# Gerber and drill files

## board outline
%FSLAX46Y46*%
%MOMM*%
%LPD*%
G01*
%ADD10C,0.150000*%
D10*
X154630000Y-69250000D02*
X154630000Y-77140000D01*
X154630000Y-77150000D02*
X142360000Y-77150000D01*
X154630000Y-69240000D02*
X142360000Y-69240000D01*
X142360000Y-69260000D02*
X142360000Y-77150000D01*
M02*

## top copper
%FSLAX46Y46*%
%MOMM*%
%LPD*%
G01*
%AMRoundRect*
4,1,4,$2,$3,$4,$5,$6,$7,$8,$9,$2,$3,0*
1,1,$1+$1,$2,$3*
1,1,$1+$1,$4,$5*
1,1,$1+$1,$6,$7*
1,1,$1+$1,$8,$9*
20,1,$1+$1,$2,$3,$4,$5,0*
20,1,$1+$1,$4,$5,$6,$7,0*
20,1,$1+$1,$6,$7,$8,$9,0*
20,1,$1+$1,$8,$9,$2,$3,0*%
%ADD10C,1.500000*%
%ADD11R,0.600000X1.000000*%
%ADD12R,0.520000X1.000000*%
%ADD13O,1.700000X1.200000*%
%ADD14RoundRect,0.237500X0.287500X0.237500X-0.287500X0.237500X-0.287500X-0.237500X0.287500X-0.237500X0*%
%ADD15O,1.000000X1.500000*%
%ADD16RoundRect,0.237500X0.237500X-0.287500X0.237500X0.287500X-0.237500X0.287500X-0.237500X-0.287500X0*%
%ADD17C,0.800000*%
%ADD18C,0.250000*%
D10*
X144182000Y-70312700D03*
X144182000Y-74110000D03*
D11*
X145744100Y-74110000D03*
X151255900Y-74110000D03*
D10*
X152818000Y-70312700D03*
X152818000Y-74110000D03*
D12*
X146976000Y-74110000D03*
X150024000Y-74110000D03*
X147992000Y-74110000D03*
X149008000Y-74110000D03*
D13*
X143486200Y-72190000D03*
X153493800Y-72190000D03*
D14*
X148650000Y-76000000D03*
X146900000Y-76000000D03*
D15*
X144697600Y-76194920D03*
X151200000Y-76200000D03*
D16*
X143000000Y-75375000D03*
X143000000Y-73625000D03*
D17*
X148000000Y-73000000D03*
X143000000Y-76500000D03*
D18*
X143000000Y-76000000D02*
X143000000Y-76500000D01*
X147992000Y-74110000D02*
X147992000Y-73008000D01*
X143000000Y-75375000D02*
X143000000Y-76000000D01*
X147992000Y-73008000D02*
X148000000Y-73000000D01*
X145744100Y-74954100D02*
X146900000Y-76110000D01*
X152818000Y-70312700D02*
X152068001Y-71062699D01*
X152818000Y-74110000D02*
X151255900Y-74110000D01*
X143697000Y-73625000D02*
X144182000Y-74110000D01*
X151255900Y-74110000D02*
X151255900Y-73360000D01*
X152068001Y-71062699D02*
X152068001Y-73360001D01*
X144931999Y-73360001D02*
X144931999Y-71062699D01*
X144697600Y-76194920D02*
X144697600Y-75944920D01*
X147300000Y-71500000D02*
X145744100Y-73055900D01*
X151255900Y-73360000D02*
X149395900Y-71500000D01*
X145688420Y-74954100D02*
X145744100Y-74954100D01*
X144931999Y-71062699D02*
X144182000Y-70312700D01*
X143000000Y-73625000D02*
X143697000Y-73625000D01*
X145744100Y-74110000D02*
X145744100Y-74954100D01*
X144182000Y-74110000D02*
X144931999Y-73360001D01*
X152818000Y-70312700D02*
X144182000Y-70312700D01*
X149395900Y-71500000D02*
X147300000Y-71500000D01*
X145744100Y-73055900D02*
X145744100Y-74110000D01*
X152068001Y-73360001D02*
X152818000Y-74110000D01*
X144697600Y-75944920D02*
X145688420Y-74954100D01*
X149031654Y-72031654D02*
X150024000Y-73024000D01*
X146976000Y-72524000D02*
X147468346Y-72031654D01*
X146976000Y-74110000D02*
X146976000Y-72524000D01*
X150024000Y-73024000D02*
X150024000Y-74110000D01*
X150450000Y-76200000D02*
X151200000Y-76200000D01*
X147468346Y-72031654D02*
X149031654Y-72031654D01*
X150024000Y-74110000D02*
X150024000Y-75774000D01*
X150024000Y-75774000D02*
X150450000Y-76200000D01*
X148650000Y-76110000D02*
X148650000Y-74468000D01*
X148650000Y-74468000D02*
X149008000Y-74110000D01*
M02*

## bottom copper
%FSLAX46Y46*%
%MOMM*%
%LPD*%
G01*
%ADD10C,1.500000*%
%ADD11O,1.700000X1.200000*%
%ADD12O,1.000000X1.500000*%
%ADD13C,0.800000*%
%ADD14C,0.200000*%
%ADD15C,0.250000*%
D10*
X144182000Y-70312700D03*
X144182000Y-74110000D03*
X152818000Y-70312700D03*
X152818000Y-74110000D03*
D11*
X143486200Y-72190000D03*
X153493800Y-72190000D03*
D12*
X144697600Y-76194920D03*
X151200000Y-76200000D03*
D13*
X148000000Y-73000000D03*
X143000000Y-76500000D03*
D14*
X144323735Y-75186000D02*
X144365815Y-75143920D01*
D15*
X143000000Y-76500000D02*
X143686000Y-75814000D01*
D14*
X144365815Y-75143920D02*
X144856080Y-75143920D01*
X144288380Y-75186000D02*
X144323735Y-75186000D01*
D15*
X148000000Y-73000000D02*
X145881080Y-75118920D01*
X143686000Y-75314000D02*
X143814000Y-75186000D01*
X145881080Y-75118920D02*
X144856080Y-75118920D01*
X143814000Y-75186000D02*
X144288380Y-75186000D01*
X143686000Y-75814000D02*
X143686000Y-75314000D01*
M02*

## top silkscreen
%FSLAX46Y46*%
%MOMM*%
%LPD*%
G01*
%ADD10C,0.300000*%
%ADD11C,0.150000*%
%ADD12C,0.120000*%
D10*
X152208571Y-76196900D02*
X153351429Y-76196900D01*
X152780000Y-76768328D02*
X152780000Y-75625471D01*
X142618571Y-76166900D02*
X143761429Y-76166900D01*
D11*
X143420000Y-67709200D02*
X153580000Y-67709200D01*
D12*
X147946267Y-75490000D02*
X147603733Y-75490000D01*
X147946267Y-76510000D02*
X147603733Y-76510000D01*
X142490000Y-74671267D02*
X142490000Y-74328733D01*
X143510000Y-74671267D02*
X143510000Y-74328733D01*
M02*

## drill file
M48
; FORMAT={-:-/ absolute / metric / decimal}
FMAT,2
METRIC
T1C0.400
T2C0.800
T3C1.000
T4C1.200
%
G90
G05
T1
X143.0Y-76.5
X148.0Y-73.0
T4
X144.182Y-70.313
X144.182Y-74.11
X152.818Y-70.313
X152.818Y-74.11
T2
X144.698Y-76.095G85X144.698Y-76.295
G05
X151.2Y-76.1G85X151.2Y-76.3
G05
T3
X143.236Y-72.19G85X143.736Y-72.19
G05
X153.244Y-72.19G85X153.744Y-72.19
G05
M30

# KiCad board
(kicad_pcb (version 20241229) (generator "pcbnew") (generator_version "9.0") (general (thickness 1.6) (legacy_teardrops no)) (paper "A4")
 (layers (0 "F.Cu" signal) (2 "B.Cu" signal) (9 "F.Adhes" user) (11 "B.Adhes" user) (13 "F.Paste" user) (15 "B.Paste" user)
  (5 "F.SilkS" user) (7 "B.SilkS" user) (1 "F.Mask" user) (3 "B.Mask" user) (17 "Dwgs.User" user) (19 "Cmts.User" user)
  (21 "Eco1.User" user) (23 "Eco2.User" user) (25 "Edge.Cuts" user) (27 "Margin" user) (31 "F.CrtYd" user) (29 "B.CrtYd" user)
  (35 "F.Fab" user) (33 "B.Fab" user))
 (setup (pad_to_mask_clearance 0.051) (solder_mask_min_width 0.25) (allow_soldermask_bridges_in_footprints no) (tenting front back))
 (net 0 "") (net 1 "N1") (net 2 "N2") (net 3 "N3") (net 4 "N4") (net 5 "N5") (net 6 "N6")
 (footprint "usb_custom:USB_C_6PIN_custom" (layer "F.Cu") (at 148.5 74.11)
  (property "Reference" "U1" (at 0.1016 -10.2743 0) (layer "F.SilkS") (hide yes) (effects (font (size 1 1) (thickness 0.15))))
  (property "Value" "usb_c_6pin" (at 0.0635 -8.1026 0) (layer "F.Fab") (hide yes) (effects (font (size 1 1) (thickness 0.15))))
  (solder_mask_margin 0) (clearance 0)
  (fp_line (start -5.08 -6.4008) (end 5.08 -6.4008) (stroke (width 0.15) (type solid)) (layer "F.SilkS"))
  (pad "1" thru_hole circle (at -4.318 -3.7973) (size 1.5 1.5) (drill 1.2) (layers "*.Cu" "*.Mask") (remove_unused_layers no) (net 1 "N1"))
  (pad "1" thru_hole circle (at -4.318 0) (size 1.5 1.5) (drill 1.2) (layers "*.Cu" "*.Mask") (remove_unused_layers no) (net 1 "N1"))
  (pad "1" smd rect (at -2.7559 0) (size 0.6 1) (layers "F.Cu" "F.Mask" "F.Paste") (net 1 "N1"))
  (pad "1" smd rect (at 2.7559 0) (size 0.6 1) (layers "F.Cu" "F.Mask" "F.Paste") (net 1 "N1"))
  (pad "1" thru_hole circle (at 4.318 -3.7973) (size 1.5 1.5) (drill 1.2) (layers "*.Cu" "*.Mask") (remove_unused_layers no) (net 1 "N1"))
  (pad "1" thru_hole circle (at 4.318 0) (size 1.5 1.5) (drill 1.2) (layers "*.Cu" "*.Mask") (remove_unused_layers no) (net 1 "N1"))
  (pad "2" smd rect (at -1.524 0) (size 0.52 1) (layers "F.Cu" "F.Mask" "F.Paste") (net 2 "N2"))
  (pad "2" smd rect (at 1.524 0) (size 0.52 1) (layers "F.Cu" "F.Mask" "F.Paste") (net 2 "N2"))
  (pad "3" smd rect (at -0.508 0) (size 0.52 1) (layers "F.Cu" "F.Mask" "F.Paste") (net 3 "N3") (solder_mask_margin 0)
   (solder_paste_margin 0) (solder_paste_margin_ratio 0) (clearance 0))
  (pad "4" smd rect (at 0.508 0) (size 0.52 1) (layers "F.Cu" "F.Mask" "F.Paste") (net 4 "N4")))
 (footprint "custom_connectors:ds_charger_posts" (layer "F.Cu") (at 148.49 72.19)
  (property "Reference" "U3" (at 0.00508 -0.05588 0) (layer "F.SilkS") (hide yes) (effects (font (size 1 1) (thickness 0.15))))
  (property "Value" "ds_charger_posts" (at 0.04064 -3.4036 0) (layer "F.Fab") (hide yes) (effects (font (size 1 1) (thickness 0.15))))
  (pad "1" thru_hole oval (at -5.0038 0) (size 1.7 1.2) (drill oval 1.5 1) (layers "*.Cu" "*.Mask") (remove_unused_layers no) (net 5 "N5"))
  (pad "2" thru_hole oval (at 5.0038 0) (size 1.7 1.2) (drill oval 1.5 1) (layers "*.Cu" "*.Mask") (remove_unused_layers no) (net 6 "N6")))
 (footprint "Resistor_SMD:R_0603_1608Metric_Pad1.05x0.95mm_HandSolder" (layer "F.Cu") (at 147.775 76 180)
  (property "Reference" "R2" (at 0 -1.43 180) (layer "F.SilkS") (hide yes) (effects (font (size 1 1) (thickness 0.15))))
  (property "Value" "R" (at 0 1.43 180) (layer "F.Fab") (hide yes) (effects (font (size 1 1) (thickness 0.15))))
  (fp_line (start -0.171267 0.51) (end 0.171267 0.51) (stroke (width 0.12) (type solid)) (layer "F.SilkS"))
  (fp_line (start -0.171267 -0.51) (end 0.171267 -0.51) (stroke (width 0.12) (type solid)) (layer "F.SilkS"))
  (pad "1" smd roundrect (at -0.875 0 180) (size 1.05 0.95) (layers "F.Cu" "F.Mask" "F.Paste") (roundrect_rratio 0.25) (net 4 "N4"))
  (pad "2" smd roundrect (at 0.875 0 180) (size 1.05 0.95) (layers "F.Cu" "F.Mask" "F.Paste") (roundrect_rratio 0.25) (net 1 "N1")))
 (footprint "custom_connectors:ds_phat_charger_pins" (layer "F.Cu") (at 147.44588 76.2)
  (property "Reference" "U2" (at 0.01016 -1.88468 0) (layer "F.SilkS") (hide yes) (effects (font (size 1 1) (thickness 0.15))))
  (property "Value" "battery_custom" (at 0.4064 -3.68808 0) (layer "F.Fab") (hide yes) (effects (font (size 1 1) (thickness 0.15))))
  (pad "1" thru_hole oval (at -2.74828 -0.00508) (size 1 1.5) (drill oval 0.8 1) (layers "*.Cu" "*.Mask") (remove_unused_layers no)
   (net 1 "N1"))
  (pad "2" thru_hole oval (at 3.75412 0) (size 1 1.5) (drill oval 0.8 1) (layers "*.Cu" "*.Mask") (remove_unused_layers no) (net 2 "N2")))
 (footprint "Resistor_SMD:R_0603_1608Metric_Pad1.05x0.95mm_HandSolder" (layer "F.Cu") (at 143 74.5 90)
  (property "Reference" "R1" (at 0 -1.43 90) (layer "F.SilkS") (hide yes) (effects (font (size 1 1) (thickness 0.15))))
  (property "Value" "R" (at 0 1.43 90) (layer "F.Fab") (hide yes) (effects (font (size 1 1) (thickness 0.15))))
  (fp_line (start -0.171267 -0.51) (end 0.171267 -0.51) (stroke (width 0.12) (type solid)) (layer "F.SilkS"))
  (fp_line (start -0.171267 0.51) (end 0.171267 0.51) (stroke (width 0.12) (type solid)) (layer "F.SilkS"))
  (pad "1" smd roundrect (at -0.875 0 90) (size 1.05 0.95) (layers "F.Cu" "F.Mask" "F.Paste") (roundrect_rratio 0.25) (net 3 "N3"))
  (pad "2" smd roundrect (at 0.875 0 90) (size 1.05 0.95) (layers "F.Cu" "F.Mask" "F.Paste") (roundrect_rratio 0.25) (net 1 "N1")))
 (gr_line (start 154.63 69.25) (end 154.63 77.14) (stroke (width 0.15) (type solid)) (layer "Edge.Cuts"))
 (gr_line (start 154.63 77.15) (end 142.36 77.15) (stroke (width 0.15) (type solid)) (layer "Edge.Cuts"))
 (gr_line (start 154.63 69.24) (end 142.36 69.24) (stroke (width 0.15) (type solid)) (layer "Edge.Cuts"))
 (gr_line (start 142.36 69.26) (end 142.36 77.15) (stroke (width 0.15) (type solid)) (layer "Edge.Cuts"))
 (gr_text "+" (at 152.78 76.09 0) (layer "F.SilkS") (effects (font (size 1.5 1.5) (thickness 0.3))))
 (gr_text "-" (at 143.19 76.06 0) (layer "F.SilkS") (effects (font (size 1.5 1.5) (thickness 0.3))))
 (segment (start 143 76) (end 143 76.5) (width 0.25) (layer "F.Cu") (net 3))
 (segment (start 147.992 74.11) (end 147.992 73.008) (width 0.25) (layer "F.Cu") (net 3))
 (segment (start 143 75.375) (end 143 76) (width 0.25) (layer "F.Cu") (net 3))
 (segment (start 147.992 73.008) (end 148 73) (width 0.25) (layer "F.Cu") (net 3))
 (via (at 148 73) (size 0.8) (drill 0.4) (layers "F.Cu" "B.Cu") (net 3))
 (via (at 143 76.5) (size 0.8) (drill 0.4) (layers "F.Cu" "B.Cu") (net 3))
 (segment (start 144.323735 75.186) (end 144.365815 75.14392) (width 0.2) (layer "B.Cu") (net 3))
 (segment (start 143 76.5) (end 143.686 75.814) (width 0.25) (layer "B.Cu") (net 3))
 (segment (start 144.365815 75.14392) (end 144.85608 75.14392) (width 0.2) (layer "B.Cu") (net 3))
 (segment (start 144.28838 75.186) (end 144.323735 75.186) (width 0.2) (layer "B.Cu") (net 3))
 (segment (start 148 73) (end 145.88108 75.11892) (width 0.25) (layer "B.Cu") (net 3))
 (segment (start 143.686 75.314) (end 143.814 75.186) (width 0.25) (layer "B.Cu") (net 3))
 (segment (start 145.88108 75.11892) (end 144.85608 75.11892) (width 0.25) (layer "B.Cu") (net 3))
 (segment (start 143.814 75.186) (end 144.28838 75.186) (width 0.25) (layer "B.Cu") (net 3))
 (segment (start 143.686 75.814) (end 143.686 75.314) (width 0.25) (layer "B.Cu") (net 3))
 (segment (start 145.7441 74.9541) (end 146.9 76.11) (width 0.25) (layer "F.Cu") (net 1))
 (segment (start 152.818 70.3127) (end 152.068001 71.062699) (width 0.25) (layer "F.Cu") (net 1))
 (segment (start 152.818 74.11) (end 151.2559 74.11) (width 0.25) (layer "F.Cu") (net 1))
 (segment (start 143.697 73.625) (end 144.182 74.11) (width 0.25) (layer "F.Cu") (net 1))
 (segment (start 151.2559 74.11) (end 151.2559 73.36) (width 0.25) (layer "F.Cu") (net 1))
 (segment (start 152.068001 71.062699) (end 152.068001 73.360001) (width 0.25) (layer "F.Cu") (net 1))
 (segment (start 144.931999 73.360001) (end 144.931999 71.062699) (width 0.25) (layer "F.Cu") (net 1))
 (segment (start 144.6976 76.19492) (end 144.6976 75.94492) (width 0.25) (layer "F.Cu") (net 1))
 (segment (start 147.3 71.5) (end 145.7441 73.0559) (width 0.25) (layer "F.Cu") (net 1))
 (segment (start 151.2559 73.36) (end 149.3959 71.5) (width 0.25) (layer "F.Cu") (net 1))
 (segment (start 145.68842 74.9541) (end 145.7441 74.9541) (width 0.25) (layer "F.Cu") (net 1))
 (segment (start 144.931999 71.062699) (end 144.182 70.3127) (width 0.25) (layer "F.Cu") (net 1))
 (segment (start 143 73.625) (end 143.697 73.625) (width 0.25) (layer "F.Cu") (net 1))
 (segment (start 145.7441 74.11) (end 145.7441 74.9541) (width 0.25) (layer "F.Cu") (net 1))
 (segment (start 144.182 74.11) (end 144.931999 73.360001) (width 0.25) (layer "F.Cu") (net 1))
 (segment (start 152.818 70.3127) (end 144.182 70.3127) (width 0.25) (layer "F.Cu") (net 1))
 (segment (start 149.3959 71.5) (end 147.3 71.5) (width 0.25) (layer "F.Cu") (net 1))
 (segment (start 145.7441 73.0559) (end 145.7441 74.11) (width 0.25) (layer "F.Cu") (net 1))
 (segment (start 152.068001 73.360001) (end 152.818 74.11) (width 0.25) (layer "F.Cu") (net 1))
 (segment (start 144.6976 75.94492) (end 145.68842 74.9541) (width 0.25) (layer "F.Cu") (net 1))
 (segment (start 149.031654 72.031654) (end 150.024 73.024) (width 0.25) (layer "F.Cu") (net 2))
 (segment (start 146.976 72.524) (end 147.468346 72.031654) (width 0.25) (layer "F.Cu") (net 2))
 (segment (start 146.976 74.11) (end 146.976 72.524) (width 0.25) (layer "F.Cu") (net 2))
 (segment (start 150.024 73.024) (end 150.024 74.11) (width 0.25) (layer "F.Cu") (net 2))
 (segment (start 150.45 76.2) (end 151.2 76.2) (width 0.25) (layer "F.Cu") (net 2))
 (segment (start 147.468346 72.031654) (end 149.031654 72.031654) (width 0.25) (layer "F.Cu") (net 2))
 (segment (start 150.024 74.11) (end 150.024 75.774) (width 0.25) (layer "F.Cu") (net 2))
 (segment (start 150.024 75.774) (end 150.45 76.2) (width 0.25) (layer "F.Cu") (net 2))
 (segment (start 148.65 76.11) (end 148.65 74.468) (width 0.25) (layer "F.Cu") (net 4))
 (segment (start 148.65 74.468) (end 149.008 74.11) (width 0.25) (layer "F.Cu") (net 4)))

